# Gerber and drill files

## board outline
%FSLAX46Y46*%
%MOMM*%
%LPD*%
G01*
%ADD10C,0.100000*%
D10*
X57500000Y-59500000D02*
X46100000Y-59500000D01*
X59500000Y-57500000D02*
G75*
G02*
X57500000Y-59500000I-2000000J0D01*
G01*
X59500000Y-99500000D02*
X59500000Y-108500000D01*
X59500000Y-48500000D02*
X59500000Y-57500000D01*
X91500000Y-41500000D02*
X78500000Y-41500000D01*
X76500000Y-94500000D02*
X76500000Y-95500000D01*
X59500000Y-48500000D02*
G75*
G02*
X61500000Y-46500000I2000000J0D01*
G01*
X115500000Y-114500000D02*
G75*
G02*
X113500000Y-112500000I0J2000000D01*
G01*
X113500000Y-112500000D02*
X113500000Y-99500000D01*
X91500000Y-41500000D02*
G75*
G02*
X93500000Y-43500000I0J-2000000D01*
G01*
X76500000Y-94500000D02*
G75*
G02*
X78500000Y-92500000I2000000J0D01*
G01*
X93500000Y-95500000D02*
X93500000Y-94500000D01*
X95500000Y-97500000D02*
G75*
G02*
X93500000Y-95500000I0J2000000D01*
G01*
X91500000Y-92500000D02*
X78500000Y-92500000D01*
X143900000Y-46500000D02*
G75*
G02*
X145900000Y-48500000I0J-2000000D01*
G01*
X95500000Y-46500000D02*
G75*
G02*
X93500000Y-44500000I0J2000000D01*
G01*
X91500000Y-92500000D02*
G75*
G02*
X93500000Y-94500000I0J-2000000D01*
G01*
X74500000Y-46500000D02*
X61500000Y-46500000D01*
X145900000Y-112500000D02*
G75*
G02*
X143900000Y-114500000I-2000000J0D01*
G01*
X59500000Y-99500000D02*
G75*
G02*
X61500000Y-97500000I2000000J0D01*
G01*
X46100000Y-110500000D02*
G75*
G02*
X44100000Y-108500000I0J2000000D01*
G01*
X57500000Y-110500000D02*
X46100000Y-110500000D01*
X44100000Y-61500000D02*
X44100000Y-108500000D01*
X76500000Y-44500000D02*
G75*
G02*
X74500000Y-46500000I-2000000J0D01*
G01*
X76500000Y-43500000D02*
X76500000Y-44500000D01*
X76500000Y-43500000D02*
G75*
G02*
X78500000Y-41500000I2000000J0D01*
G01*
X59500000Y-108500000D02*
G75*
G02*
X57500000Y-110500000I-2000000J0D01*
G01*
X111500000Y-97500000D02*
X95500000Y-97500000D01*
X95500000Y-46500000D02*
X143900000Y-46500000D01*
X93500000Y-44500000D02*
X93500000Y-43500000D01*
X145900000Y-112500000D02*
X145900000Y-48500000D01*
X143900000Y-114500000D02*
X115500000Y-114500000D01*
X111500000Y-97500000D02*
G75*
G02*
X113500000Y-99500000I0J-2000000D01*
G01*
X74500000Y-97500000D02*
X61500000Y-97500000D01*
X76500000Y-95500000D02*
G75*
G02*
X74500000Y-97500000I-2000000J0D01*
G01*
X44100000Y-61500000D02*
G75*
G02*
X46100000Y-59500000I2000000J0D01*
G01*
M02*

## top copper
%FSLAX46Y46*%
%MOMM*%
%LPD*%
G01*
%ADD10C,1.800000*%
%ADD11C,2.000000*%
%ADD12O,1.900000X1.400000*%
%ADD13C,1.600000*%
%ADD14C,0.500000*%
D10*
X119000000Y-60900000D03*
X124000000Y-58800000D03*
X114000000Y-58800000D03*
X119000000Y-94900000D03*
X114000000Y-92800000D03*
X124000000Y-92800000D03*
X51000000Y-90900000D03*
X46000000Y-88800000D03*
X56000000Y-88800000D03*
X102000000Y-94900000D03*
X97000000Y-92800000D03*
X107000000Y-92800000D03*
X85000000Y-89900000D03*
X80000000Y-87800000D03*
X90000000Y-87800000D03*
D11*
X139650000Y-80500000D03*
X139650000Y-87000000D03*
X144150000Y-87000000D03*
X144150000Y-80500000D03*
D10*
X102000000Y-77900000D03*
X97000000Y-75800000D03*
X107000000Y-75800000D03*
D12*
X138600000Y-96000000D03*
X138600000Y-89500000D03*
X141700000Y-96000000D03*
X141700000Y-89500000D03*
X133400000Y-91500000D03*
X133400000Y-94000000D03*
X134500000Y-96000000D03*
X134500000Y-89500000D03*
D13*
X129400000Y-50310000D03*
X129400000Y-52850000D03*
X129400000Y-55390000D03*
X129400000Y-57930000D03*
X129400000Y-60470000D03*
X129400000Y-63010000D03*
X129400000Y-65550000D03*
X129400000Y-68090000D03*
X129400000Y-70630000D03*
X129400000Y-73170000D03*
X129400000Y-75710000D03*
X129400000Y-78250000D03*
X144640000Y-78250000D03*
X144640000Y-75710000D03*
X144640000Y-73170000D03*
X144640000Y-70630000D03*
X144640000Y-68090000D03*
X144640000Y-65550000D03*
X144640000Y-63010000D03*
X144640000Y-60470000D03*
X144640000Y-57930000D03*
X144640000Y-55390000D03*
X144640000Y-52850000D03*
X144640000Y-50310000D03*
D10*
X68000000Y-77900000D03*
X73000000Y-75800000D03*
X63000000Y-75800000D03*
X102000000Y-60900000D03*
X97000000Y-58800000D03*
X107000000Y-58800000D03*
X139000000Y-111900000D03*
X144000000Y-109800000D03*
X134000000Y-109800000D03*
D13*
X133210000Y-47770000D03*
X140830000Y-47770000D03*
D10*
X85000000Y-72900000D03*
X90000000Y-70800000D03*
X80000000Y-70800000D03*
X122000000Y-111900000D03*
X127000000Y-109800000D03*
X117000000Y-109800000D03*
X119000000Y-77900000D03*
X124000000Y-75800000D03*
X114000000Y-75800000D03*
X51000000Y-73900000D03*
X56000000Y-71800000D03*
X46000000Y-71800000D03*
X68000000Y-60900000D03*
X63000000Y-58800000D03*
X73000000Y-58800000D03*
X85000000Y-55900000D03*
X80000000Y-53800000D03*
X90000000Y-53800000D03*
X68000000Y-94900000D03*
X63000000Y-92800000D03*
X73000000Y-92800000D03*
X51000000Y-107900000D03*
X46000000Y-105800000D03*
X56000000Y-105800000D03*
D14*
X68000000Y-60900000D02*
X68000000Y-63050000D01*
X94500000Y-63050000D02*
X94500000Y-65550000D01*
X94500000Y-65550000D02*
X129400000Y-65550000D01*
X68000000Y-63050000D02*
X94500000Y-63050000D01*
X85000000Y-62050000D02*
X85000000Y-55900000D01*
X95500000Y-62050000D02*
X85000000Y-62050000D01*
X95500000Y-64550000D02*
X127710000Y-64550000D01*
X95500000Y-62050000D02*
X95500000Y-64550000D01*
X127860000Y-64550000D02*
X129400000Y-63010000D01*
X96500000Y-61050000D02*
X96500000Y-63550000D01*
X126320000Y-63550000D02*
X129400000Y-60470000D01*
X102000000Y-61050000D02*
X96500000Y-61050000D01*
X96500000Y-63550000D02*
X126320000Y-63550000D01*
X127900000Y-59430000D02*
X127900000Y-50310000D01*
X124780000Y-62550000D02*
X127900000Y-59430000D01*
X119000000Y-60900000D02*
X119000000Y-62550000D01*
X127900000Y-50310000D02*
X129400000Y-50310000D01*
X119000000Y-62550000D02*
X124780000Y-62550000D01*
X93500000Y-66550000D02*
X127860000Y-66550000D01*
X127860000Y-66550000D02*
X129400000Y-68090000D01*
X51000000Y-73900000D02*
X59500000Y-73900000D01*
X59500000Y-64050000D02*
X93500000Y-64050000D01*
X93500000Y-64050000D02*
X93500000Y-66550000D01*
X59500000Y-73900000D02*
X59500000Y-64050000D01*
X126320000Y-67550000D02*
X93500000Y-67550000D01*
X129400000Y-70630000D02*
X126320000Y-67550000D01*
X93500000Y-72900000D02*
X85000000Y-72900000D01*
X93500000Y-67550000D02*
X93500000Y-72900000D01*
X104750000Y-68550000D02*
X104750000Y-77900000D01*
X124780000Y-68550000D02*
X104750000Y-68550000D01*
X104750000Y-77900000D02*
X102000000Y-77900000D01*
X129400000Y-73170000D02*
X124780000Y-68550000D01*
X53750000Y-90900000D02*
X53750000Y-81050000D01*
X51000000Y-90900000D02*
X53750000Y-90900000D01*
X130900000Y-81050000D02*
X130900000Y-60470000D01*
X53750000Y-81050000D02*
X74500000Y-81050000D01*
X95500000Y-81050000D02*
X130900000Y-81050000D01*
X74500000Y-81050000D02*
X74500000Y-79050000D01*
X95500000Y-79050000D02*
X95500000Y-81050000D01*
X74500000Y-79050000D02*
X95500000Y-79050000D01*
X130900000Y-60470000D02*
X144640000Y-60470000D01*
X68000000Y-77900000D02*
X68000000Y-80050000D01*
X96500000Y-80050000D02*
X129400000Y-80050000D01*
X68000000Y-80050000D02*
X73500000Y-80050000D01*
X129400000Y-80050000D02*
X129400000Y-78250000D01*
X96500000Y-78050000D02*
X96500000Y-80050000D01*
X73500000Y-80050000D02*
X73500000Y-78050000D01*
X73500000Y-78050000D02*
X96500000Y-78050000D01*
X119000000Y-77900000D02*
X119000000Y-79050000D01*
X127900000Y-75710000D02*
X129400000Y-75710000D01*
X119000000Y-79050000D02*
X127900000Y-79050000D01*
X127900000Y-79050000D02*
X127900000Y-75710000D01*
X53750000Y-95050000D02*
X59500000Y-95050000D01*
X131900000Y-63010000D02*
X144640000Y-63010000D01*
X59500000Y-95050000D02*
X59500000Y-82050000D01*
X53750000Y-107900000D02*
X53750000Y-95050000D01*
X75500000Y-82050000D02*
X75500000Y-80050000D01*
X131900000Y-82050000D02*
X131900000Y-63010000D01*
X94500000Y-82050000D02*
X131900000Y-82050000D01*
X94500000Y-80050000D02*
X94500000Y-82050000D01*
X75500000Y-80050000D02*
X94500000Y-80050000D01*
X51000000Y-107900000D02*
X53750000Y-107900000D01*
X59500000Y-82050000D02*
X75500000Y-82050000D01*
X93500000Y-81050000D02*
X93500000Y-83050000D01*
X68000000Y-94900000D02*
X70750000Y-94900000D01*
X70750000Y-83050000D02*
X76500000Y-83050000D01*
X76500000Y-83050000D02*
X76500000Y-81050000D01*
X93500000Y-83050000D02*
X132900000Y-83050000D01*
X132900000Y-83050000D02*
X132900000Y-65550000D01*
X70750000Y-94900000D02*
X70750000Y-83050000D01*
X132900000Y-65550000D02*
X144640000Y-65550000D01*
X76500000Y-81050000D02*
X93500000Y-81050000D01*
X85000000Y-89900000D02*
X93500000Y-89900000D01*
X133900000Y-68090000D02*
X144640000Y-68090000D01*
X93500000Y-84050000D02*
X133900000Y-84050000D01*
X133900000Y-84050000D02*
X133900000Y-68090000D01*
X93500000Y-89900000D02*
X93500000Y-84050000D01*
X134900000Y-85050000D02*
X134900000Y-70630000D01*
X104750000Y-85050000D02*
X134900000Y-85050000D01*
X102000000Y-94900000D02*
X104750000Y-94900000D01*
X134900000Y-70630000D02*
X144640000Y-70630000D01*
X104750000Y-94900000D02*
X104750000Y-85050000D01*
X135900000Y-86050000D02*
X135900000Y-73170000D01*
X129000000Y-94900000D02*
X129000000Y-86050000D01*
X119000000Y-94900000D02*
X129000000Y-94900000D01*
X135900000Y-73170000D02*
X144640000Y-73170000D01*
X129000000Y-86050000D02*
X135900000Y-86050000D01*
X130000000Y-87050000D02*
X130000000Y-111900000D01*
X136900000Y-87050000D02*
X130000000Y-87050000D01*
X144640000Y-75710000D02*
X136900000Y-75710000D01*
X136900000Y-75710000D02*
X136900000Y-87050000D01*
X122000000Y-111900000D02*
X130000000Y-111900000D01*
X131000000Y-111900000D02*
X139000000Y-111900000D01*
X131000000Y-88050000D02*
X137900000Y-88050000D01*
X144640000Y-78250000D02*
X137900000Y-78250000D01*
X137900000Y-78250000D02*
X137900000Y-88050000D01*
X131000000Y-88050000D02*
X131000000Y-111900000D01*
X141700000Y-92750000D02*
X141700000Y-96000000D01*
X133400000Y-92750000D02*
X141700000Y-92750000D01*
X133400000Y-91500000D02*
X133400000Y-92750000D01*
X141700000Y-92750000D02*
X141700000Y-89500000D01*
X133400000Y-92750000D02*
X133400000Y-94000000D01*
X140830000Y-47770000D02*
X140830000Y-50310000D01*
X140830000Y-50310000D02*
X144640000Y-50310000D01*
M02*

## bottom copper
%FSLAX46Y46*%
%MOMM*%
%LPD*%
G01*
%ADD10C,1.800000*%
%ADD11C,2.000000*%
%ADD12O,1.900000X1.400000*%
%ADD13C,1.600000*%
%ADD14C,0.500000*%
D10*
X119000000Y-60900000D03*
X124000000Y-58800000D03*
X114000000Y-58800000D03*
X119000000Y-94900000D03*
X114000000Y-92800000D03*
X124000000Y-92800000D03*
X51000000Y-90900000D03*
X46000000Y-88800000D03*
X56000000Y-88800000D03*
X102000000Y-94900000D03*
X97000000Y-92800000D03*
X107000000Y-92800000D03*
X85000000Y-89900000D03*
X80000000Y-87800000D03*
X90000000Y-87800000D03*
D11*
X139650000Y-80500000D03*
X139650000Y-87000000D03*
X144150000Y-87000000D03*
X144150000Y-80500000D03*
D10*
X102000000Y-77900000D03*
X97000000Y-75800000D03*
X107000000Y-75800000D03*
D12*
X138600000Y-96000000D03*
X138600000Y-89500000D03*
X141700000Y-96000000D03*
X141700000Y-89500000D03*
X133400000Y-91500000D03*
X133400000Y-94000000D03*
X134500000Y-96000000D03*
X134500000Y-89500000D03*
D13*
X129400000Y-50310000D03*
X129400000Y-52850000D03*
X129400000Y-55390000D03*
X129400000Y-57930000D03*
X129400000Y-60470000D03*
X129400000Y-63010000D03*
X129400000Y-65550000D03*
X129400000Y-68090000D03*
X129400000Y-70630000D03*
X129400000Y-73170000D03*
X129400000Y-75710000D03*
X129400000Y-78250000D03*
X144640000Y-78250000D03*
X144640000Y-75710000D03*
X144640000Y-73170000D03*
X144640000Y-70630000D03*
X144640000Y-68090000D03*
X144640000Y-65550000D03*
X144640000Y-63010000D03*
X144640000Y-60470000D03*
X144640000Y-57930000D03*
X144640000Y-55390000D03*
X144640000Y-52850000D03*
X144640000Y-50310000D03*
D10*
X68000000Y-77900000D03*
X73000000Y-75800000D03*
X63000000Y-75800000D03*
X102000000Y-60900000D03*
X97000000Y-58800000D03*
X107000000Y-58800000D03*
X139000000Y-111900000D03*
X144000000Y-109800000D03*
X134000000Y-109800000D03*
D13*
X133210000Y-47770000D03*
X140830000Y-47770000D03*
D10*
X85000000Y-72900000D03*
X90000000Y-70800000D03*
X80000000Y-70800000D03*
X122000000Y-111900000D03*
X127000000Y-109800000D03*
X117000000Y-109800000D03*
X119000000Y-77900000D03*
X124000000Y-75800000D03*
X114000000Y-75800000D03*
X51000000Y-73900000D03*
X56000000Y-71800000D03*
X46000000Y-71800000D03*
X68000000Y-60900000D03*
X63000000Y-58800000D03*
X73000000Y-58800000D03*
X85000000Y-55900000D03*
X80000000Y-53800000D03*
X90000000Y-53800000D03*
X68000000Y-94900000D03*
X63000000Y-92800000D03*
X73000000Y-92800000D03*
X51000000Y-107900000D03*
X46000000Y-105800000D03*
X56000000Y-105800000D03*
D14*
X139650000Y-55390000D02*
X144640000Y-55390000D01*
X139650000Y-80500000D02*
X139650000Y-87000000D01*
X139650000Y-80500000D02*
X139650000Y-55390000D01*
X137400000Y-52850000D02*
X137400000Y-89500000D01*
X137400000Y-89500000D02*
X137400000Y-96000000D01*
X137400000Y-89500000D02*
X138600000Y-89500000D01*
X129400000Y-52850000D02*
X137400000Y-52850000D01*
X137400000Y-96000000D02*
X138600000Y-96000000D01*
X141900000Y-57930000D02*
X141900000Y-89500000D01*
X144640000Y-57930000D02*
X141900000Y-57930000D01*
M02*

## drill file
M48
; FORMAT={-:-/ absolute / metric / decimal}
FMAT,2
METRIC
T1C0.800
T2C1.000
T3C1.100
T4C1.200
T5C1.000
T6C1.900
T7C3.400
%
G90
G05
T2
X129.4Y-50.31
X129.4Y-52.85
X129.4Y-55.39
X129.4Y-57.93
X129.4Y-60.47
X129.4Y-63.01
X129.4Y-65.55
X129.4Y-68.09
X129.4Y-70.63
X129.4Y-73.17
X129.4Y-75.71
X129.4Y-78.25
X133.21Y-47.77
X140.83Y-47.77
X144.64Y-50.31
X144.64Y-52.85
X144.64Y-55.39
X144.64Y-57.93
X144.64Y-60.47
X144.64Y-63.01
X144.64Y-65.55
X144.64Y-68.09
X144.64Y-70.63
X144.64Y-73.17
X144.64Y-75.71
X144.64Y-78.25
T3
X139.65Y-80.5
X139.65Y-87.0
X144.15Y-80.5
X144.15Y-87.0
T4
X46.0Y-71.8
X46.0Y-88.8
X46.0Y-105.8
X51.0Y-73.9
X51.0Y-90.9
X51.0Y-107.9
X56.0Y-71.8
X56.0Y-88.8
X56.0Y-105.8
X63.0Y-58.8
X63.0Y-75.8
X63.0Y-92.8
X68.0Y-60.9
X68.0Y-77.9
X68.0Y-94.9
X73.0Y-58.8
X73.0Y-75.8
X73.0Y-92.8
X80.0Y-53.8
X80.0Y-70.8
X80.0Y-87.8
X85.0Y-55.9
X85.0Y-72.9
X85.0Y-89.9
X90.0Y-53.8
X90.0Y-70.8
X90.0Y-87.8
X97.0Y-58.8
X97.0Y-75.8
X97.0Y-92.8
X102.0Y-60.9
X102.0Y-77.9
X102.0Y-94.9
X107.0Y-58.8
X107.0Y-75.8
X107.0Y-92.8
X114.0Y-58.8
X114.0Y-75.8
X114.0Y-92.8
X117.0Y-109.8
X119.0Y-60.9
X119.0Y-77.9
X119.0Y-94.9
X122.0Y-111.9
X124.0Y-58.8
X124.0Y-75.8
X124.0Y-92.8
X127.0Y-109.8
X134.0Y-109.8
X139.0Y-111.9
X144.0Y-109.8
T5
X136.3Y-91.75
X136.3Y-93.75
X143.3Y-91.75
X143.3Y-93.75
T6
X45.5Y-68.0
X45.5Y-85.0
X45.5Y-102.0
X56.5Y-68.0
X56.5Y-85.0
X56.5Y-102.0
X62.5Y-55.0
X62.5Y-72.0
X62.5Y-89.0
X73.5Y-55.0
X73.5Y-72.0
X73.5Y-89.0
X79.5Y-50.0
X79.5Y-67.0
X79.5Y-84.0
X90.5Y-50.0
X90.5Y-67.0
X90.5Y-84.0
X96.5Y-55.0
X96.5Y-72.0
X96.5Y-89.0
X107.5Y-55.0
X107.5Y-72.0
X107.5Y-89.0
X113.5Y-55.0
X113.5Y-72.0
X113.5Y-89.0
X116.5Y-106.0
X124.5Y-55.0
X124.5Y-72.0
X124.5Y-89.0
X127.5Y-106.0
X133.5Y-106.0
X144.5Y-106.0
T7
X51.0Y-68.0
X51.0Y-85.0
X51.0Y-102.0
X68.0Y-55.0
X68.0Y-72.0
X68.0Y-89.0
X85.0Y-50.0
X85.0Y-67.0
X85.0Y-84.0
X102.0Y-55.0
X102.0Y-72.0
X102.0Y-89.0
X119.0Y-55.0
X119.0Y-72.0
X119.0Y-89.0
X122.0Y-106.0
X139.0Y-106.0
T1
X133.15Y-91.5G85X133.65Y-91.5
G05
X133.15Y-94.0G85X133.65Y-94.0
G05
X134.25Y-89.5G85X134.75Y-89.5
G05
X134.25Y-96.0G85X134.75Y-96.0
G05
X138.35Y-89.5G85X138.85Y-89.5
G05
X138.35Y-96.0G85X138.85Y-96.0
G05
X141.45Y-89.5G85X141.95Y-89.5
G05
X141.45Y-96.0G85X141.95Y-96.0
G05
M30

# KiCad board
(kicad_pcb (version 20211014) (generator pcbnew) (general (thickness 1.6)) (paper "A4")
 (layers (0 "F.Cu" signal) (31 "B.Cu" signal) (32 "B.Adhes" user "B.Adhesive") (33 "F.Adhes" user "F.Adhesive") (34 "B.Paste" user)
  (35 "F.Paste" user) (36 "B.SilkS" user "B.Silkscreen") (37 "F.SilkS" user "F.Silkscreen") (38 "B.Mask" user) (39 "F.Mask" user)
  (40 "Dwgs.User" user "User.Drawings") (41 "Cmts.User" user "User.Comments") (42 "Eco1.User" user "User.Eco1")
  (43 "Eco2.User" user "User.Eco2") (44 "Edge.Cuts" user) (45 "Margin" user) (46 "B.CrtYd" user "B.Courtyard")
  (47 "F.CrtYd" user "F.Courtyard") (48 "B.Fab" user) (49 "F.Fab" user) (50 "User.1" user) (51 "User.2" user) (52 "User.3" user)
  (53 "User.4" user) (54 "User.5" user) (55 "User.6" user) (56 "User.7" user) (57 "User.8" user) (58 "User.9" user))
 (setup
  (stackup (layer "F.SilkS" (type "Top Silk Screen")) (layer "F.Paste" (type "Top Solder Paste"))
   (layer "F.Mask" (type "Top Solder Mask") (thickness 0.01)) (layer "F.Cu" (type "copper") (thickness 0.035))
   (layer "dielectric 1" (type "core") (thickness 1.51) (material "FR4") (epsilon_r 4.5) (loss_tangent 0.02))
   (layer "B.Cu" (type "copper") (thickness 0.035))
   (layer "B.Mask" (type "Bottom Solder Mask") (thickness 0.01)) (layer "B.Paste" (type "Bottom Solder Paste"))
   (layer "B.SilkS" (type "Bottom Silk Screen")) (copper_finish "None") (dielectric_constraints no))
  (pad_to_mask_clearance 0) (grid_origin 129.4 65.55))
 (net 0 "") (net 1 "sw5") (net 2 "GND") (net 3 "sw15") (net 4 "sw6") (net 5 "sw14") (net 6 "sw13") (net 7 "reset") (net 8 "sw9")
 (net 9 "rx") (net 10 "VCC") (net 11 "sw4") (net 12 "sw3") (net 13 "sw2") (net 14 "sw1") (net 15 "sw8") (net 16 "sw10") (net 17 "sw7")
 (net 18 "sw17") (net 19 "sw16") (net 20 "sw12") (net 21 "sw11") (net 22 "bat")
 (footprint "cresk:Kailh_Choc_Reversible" (layer "F.Cu") (at 119 55)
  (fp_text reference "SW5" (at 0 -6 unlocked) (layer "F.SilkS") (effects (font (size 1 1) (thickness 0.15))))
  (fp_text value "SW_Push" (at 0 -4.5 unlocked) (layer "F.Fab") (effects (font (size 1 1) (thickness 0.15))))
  (pad "" np_thru_hole circle (at 0 0) (size 3.4 3.4) (drill 3.4) (layers *.Mask))
  (pad "" np_thru_hole circle (at -5.5 0) (size 1.9 1.9) (drill 1.9) (layers *.Mask))
  (pad "" np_thru_hole circle (at 5.5 0) (size 1.9 1.9) (drill 1.9) (layers *.Mask))
  (pad "1" thru_hole circle (at 0 5.9) (size 1.8 1.8) (drill 1.2) (layers *.Cu *.Mask) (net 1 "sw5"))
  (pad "2" thru_hole circle (at 5 3.8) (size 1.8 1.8) (drill 1.2) (layers *.Cu *.Mask) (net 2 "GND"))
  (pad "2" thru_hole circle (at -5 3.8) (size 1.8 1.8) (drill 1.2) (layers *.Cu *.Mask) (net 2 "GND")))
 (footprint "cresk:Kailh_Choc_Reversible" (layer "F.Cu") (at 119 89)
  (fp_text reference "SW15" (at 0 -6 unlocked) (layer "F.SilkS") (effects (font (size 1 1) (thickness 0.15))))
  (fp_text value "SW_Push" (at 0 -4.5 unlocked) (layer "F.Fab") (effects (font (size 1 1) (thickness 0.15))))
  (pad "" np_thru_hole circle (at 5.5 0) (size 1.9 1.9) (drill 1.9) (layers *.Mask))
  (pad "" np_thru_hole circle (at 0 0) (size 3.4 3.4) (drill 3.4) (layers *.Mask))
  (pad "" np_thru_hole circle (at -5.5 0) (size 1.9 1.9) (drill 1.9) (layers *.Mask))
  (pad "1" thru_hole circle (at 0 5.9) (size 1.8 1.8) (drill 1.2) (layers *.Cu *.Mask) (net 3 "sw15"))
  (pad "2" thru_hole circle (at -5 3.8) (size 1.8 1.8) (drill 1.2) (layers *.Cu *.Mask) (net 2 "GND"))
  (pad "2" thru_hole circle (at 5 3.8) (size 1.8 1.8) (drill 1.2) (layers *.Cu *.Mask) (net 2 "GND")))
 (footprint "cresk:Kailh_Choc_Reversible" (layer "F.Cu") (at 51 85)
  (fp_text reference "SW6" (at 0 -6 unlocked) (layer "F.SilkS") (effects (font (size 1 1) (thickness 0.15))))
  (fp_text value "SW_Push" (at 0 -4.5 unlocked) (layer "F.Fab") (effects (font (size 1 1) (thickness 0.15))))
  (pad "" np_thru_hole circle (at 0 0) (size 3.4 3.4) (drill 3.4) (layers *.Mask))
  (pad "" np_thru_hole circle (at 5.5 0) (size 1.9 1.9) (drill 1.9) (layers *.Mask))
  (pad "" np_thru_hole circle (at -5.5 0) (size 1.9 1.9) (drill 1.9) (layers *.Mask))
  (pad "1" thru_hole circle (at 0 5.9) (size 1.8 1.8) (drill 1.2) (layers *.Cu *.Mask) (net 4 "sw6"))
  (pad "2" thru_hole circle (at -5 3.8) (size 1.8 1.8) (drill 1.2) (layers *.Cu *.Mask) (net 2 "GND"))
  (pad "2" thru_hole circle (at 5 3.8) (size 1.8 1.8) (drill 1.2) (layers *.Cu *.Mask) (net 2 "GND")))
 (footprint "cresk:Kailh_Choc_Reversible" (layer "F.Cu") (at 102 89)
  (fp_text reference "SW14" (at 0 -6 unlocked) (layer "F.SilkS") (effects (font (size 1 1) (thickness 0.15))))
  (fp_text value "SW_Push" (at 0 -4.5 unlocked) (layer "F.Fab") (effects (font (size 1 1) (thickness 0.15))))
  (pad "" np_thru_hole circle (at -5.5 0) (size 1.9 1.9) (drill 1.9) (layers *.Mask))
  (pad "" np_thru_hole circle (at 0 0) (size 3.4 3.4) (drill 3.4) (layers *.Mask))
  (pad "" np_thru_hole circle (at 5.5 0) (size 1.9 1.9) (drill 1.9) (layers *.Mask))
  (pad "1" thru_hole circle (at 0 5.9) (size 1.8 1.8) (drill 1.2) (layers *.Cu *.Mask) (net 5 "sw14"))
  (pad "2" thru_hole circle (at -5 3.8) (size 1.8 1.8) (drill 1.2) (layers *.Cu *.Mask) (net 2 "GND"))
  (pad "2" thru_hole circle (at 5 3.8) (size 1.8 1.8) (drill 1.2) (layers *.Cu *.Mask) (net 2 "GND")))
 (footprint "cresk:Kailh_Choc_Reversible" (layer "F.Cu") (at 85 84)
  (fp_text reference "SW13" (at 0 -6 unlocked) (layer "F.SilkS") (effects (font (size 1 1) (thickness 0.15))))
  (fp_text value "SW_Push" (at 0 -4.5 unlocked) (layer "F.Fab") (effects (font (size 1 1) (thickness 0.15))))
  (pad "" np_thru_hole circle (at 0 0) (size 3.4 3.4) (drill 3.4) (layers *.Mask))
  (pad "" np_thru_hole circle (at -5.5 0) (size 1.9 1.9) (drill 1.9) (layers *.Mask))
  (pad "" np_thru_hole circle (at 5.5 0) (size 1.9 1.9) (drill 1.9) (layers *.Mask))
  (pad "1" thru_hole circle (at 0 5.9) (size 1.8 1.8) (drill 1.2) (layers *.Cu *.Mask) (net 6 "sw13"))
  (pad "2" thru_hole circle (at -5 3.8) (size 1.8 1.8) (drill 1.2) (layers *.Cu *.Mask) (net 2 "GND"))
  (pad "2" thru_hole circle (at 5 3.8) (size 1.8 1.8) (drill 1.2) (layers *.Cu *.Mask) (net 2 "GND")))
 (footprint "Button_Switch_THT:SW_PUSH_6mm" (layer "F.Cu") (at 139.65 87 90)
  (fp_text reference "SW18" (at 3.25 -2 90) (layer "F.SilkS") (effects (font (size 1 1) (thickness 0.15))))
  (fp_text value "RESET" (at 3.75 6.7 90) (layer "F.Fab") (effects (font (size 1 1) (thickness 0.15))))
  (pad "1" thru_hole circle (at 6.5 0 180) (size 2 2) (drill 1.1) (layers *.Cu *.Mask) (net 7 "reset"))
  (pad "1" thru_hole circle (at 0 0 180) (size 2 2) (drill 1.1) (layers *.Cu *.Mask) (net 7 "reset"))
  (pad "2" thru_hole circle (at 0 4.5 180) (size 2 2) (drill 1.1) (layers *.Cu *.Mask) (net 2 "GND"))
  (pad "2" thru_hole circle (at 6.5 4.5 180) (size 2 2) (drill 1.1) (layers *.Cu *.Mask) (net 2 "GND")))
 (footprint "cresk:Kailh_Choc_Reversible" (layer "F.Cu") (at 102 72)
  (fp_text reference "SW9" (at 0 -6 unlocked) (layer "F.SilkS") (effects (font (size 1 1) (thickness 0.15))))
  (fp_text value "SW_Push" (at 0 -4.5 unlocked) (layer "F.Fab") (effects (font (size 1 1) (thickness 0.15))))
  (pad "" np_thru_hole circle (at -5.5 0) (size 1.9 1.9) (drill 1.9) (layers *.Mask))
  (pad "" np_thru_hole circle (at 0 0) (size 3.4 3.4) (drill 3.4) (layers *.Mask))
  (pad "" np_thru_hole circle (at 5.5 0) (size 1.9 1.9) (drill 1.9) (layers *.Mask))
  (pad "1" thru_hole circle (at 0 5.9) (size 1.8 1.8) (drill 1.2) (layers *.Cu *.Mask) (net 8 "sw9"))
  (pad "2" thru_hole circle (at -5 3.8) (size 1.8 1.8) (drill 1.2) (layers *.Cu *.Mask) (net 2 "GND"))
  (pad "2" thru_hole circle (at 5 3.8) (size 1.8 1.8) (drill 1.2) (layers *.Cu *.Mask) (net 2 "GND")))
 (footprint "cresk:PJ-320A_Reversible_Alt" (layer "F.Cu") (at 133.4 96 90)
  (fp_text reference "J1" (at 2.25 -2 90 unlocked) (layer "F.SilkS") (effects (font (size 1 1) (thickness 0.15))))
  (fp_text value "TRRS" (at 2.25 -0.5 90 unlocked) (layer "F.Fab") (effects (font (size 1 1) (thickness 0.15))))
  (pad "" np_thru_hole circle (at 2.25 2.9 90) (size 1 1) (drill 1) (layers *.Mask))
  (pad "" np_thru_hole circle (at 4.25 2.9 90) (size 1 1) (drill 1) (layers *.Mask))
  (pad "" np_thru_hole circle (at 2.25 9.9 90) (size 1 1) (drill 1) (layers *.Mask))
  (pad "" np_thru_hole circle (at 4.25 9.9 90) (size 1 1) (drill 1) (layers *.Mask))
  (pad "R1" thru_hole oval (at 0 5.2 90) (size 1.4 1.9) (drill oval 0.8 1.3) (layers *.Cu *.Mask) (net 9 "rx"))
  (pad "R1" thru_hole oval (at 6.5 5.2 90) (size 1.4 1.9) (drill oval 0.8 1.3) (layers *.Cu *.Mask) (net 9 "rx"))
  (pad "R2" thru_hole oval (at 0 8.3 90) (size 1.4 1.9) (drill oval 0.8 1.3) (layers *.Cu *.Mask) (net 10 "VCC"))
  (pad "R2" thru_hole oval (at 6.5 8.3 90) (size 1.4 1.9) (drill oval 0.8 1.3) (layers *.Cu *.Mask) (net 10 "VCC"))
  (pad "S" thru_hole oval (at 4.5 0 90) (size 1.4 1.9) (drill oval 0.8 1.3) (layers *.Cu *.Mask) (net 10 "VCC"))
  (pad "S" thru_hole oval (at 2 0 90) (size 1.4 1.9) (drill oval 0.8 1.3) (layers *.Cu *.Mask) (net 10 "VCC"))
  (pad "T" thru_hole oval (at 0 1.1 90) (size 1.4 1.9) (drill oval 0.8 1.3) (layers *.Cu *.Mask) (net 2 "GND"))
  (pad "T" thru_hole oval (at 6.5 1.1 90) (size 1.4 1.9) (drill oval 0.8 1.3) (layers *.Cu *.Mask) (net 2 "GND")))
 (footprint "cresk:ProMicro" (layer "F.Cu") (at 129.4 50.31)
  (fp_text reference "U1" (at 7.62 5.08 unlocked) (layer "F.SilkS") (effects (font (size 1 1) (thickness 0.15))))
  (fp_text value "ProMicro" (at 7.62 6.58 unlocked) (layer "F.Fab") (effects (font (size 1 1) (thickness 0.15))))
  (pad "1" thru_hole circle (at 0 0) (size 1.6 1.6) (drill 1) (layers *.Cu *.Mask) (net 1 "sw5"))
  (pad "2" thru_hole circle (at 0 2.54) (size 1.6 1.6) (drill 1) (layers *.Cu *.Mask) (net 9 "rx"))
  (pad "3" thru_hole circle (at 0 5.08) (size 1.6 1.6) (drill 1) (layers *.Cu *.Mask) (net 2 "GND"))
  (pad "4" thru_hole circle (at 0 7.62) (size 1.6 1.6) (drill 1) (layers *.Cu *.Mask) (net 2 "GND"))
  (pad "5" thru_hole circle (at 0 10.16) (size 1.6 1.6) (drill 1) (layers *.Cu *.Mask) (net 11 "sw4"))
  (pad "6" thru_hole circle (at 0 12.7) (size 1.6 1.6) (drill 1) (layers *.Cu *.Mask) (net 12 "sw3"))
  (pad "7" thru_hole circle (at 0 15.24) (size 1.6 1.6) (drill 1) (layers *.Cu *.Mask) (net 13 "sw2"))
  (pad "8" thru_hole circle (at 0 17.78) (size 1.6 1.6) (drill 1) (layers *.Cu *.Mask) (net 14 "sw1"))
  (pad "9" thru_hole circle (at 0 20.32) (size 1.6 1.6) (drill 1) (layers *.Cu *.Mask) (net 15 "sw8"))
  (pad "10" thru_hole circle (at 0 22.86) (size 1.6 1.6) (drill 1) (layers *.Cu *.Mask) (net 8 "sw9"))
  (pad "11" thru_hole circle (at 0 25.4) (size 1.6 1.6) (drill 1) (layers *.Cu *.Mask) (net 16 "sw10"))
  (pad "12" thru_hole circle (at 0 27.94) (size 1.6 1.6) (drill 1) (layers *.Cu *.Mask) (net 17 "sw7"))
  (pad "13" thru_hole circle (at 15.24 27.94) (size 1.6 1.6) (drill 1) (layers *.Cu *.Mask) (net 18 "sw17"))
  (pad "14" thru_hole circle (at 15.24 25.4) (size 1.6 1.6) (drill 1) (layers *.Cu *.Mask) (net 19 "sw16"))
  (pad "15" thru_hole circle (at 15.24 22.86) (size 1.6 1.6) (drill 1) (layers *.Cu *.Mask) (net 3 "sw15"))
  (pad "16" thru_hole circle (at 15.24 20.32) (size 1.6 1.6) (drill 1) (layers *.Cu *.Mask) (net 5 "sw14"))
  (pad "17" thru_hole circle (at 15.24 17.78) (size 1.6 1.6) (drill 1) (layers *.Cu *.Mask) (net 6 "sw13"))
  (pad "18" thru_hole circle (at 15.24 15.24) (size 1.6 1.6) (drill 1) (layers *.Cu *.Mask) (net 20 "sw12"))
  (pad "19" thru_hole circle (at 15.24 12.7) (size 1.6 1.6) (drill 1) (layers *.Cu *.Mask) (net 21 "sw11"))
  (pad "20" thru_hole circle (at 15.24 10.16) (size 1.6 1.6) (drill 1) (layers *.Cu *.Mask) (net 4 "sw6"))
  (pad "21" thru_hole circle (at 15.24 7.62) (size 1.6 1.6) (drill 1) (layers *.Cu *.Mask) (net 10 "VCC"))
  (pad "22" thru_hole circle (at 15.24 5.08) (size 1.6 1.6) (drill 1) (layers *.Cu *.Mask) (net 7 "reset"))
  (pad "23" thru_hole circle (at 15.24 2.54) (size 1.6 1.6) (drill 1) (layers *.Cu *.Mask) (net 2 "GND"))
  (pad "24" thru_hole circle (at 15.24 0) (size 1.6 1.6) (drill 1) (layers *.Cu *.Mask) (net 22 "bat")))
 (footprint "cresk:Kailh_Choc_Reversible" (layer "F.Cu") (at 68 72)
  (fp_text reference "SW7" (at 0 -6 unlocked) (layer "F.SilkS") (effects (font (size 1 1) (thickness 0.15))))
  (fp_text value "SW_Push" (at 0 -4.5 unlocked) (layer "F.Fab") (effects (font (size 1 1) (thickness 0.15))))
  (pad "" np_thru_hole circle (at 5.5 0) (size 1.9 1.9) (drill 1.9) (layers *.Mask))
  (pad "" np_thru_hole circle (at -5.5 0) (size 1.9 1.9) (drill 1.9) (layers *.Mask))
  (pad "" np_thru_hole circle (at 0 0) (size 3.4 3.4) (drill 3.4) (layers *.Mask))
  (pad "1" thru_hole circle (at 0 5.9) (size 1.8 1.8) (drill 1.2) (layers *.Cu *.Mask) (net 17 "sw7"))
  (pad "2" thru_hole circle (at 5 3.8) (size 1.8 1.8) (drill 1.2) (layers *.Cu *.Mask) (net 2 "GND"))
  (pad "2" thru_hole circle (at -5 3.8) (size 1.8 1.8) (drill 1.2) (layers *.Cu *.Mask) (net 2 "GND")))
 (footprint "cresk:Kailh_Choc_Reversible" (layer "F.Cu") (at 102 55)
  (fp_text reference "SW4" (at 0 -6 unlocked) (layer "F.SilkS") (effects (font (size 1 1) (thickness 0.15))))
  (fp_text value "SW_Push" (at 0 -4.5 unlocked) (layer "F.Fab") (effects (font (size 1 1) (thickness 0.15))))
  (pad "" np_thru_hole circle (at 5.5 0) (size 1.9 1.9) (drill 1.9) (layers *.Mask))
  (pad "" np_thru_hole circle (at -5.5 0) (size 1.9 1.9) (drill 1.9) (layers *.Mask))
  (pad "" np_thru_hole circle (at 0 0) (size 3.4 3.4) (drill 3.4) (layers *.Mask))
  (pad "1" thru_hole circle (at 0 5.9) (size 1.8 1.8) (drill 1.2) (layers *.Cu *.Mask) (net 11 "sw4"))
  (pad "2" thru_hole circle (at -5 3.8) (size 1.8 1.8) (drill 1.2) (layers *.Cu *.Mask) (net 2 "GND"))
  (pad "2" thru_hole circle (at 5 3.8) (size 1.8 1.8) (drill 1.2) (layers *.Cu *.Mask) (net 2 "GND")))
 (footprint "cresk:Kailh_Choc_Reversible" (layer "F.Cu") (at 139 106)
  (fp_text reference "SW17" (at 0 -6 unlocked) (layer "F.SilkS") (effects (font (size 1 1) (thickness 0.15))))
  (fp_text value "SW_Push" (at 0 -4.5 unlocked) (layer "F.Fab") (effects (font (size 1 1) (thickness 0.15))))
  (pad "" np_thru_hole circle (at -5.5 0) (size 1.9 1.9) (drill 1.9) (layers *.Mask))
  (pad "" np_thru_hole circle (at 5.5 0) (size 1.9 1.9) (drill 1.9) (layers *.Mask))
  (pad "" np_thru_hole circle (at 0 0) (size 3.4 3.4) (drill 3.4) (layers *.Mask))
  (pad "1" thru_hole circle (at 0 5.9) (size 1.8 1.8) (drill 1.2) (layers *.Cu *.Mask) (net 18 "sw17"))
  (pad "2" thru_hole circle (at 5 3.8) (size 1.8 1.8) (drill 1.2) (layers *.Cu *.Mask) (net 2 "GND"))
  (pad "2" thru_hole circle (at -5 3.8) (size 1.8 1.8) (drill 1.2) (layers *.Cu *.Mask) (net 2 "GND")))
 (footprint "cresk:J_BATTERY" (layer "F.Cu") (at 133.21 47.77)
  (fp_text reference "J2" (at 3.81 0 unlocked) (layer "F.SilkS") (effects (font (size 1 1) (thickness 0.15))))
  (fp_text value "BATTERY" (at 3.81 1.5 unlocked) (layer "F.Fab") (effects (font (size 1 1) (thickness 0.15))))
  (pad "1" thru_hole circle (at 0 0) (size 1.6 1.6) (drill 1) (layers *.Cu *.Mask) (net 2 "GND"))
  (pad "2" thru_hole circle (at 7.62 0) (size 1.6 1.6) (drill 1) (layers *.Cu *.Mask) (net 22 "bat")))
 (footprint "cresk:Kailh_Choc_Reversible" (layer "F.Cu") (at 85 67)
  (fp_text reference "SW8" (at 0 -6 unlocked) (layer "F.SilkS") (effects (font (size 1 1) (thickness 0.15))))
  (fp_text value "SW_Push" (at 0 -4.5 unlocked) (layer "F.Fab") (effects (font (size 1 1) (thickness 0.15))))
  (pad "" np_thru_hole circle (at 0 0) (size 3.4 3.4) (drill 3.4) (layers *.Mask))
  (pad "" np_thru_hole circle (at -5.5 0) (size 1.9 1.9) (drill 1.9) (layers *.Mask))
  (pad "" np_thru_hole circle (at 5.5 0) (size 1.9 1.9) (drill 1.9) (layers *.Mask))
  (pad "1" thru_hole circle (at 0 5.9) (size 1.8 1.8) (drill 1.2) (layers *.Cu *.Mask) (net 15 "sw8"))
  (pad "2" thru_hole circle (at 5 3.8) (size 1.8 1.8) (drill 1.2) (layers *.Cu *.Mask) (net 2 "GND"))
  (pad "2" thru_hole circle (at -5 3.8) (size 1.8 1.8) (drill 1.2) (layers *.Cu *.Mask) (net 2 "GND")))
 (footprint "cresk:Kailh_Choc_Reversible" (layer "F.Cu") (at 122 106)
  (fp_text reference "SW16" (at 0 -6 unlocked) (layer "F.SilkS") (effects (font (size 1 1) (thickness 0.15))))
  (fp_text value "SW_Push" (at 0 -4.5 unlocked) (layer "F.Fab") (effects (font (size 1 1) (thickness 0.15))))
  (pad "" np_thru_hole circle (at 0 0) (size 3.4 3.4) (drill 3.4) (layers *.Mask))
  (pad "" np_thru_hole circle (at -5.5 0) (size 1.9 1.9) (drill 1.9) (layers *.Mask))
  (pad "" np_thru_hole circle (at 5.5 0) (size 1.9 1.9) (drill 1.9) (layers *.Mask))
  (pad "1" thru_hole circle (at 0 5.9) (size 1.8 1.8) (drill 1.2) (layers *.Cu *.Mask) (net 19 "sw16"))
  (pad "2" thru_hole circle (at 5 3.8) (size 1.8 1.8) (drill 1.2) (layers *.Cu *.Mask) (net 2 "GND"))
  (pad "2" thru_hole circle (at -5 3.8) (size 1.8 1.8) (drill 1.2) (layers *.Cu *.Mask) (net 2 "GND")))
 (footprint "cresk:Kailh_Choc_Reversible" (layer "F.Cu") (at 119 72)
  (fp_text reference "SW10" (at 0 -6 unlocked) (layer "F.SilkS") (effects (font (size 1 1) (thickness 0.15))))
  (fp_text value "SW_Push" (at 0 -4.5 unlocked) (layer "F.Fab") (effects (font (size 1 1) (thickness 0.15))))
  (pad "" np_thru_hole circle (at 0 0) (size 3.4 3.4) (drill 3.4) (layers *.Mask))
  (pad "" np_thru_hole circle (at -5.5 0) (size 1.9 1.9) (drill 1.9) (layers *.Mask))
  (pad "" np_thru_hole circle (at 5.5 0) (size 1.9 1.9) (drill 1.9) (layers *.Mask))
  (pad "1" thru_hole circle (at 0 5.9) (size 1.8 1.8) (drill 1.2) (layers *.Cu *.Mask) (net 16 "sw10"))
  (pad "2" thru_hole circle (at 5 3.8) (size 1.8 1.8) (drill 1.2) (layers *.Cu *.Mask) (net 2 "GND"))
  (pad "2" thru_hole circle (at -5 3.8) (size 1.8 1.8) (drill 1.2) (layers *.Cu *.Mask) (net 2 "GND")))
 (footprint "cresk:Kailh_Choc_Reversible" (layer "F.Cu") (at 51 68)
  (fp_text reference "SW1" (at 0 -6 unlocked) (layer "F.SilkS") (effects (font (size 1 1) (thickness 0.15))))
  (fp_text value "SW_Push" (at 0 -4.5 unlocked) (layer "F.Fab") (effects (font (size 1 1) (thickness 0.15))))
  (pad "" np_thru_hole circle (at -5.5 0) (size 1.9 1.9) (drill 1.9) (layers *.Mask))
  (pad "" np_thru_hole circle (at 5.5 0) (size 1.9 1.9) (drill 1.9) (layers *.Mask))
  (pad "" np_thru_hole circle (at 0 0) (size 3.4 3.4) (drill 3.4) (layers *.Mask))
  (pad "1" thru_hole circle (at 0 5.9) (size 1.8 1.8) (drill 1.2) (layers *.Cu *.Mask) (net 14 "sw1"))
  (pad "2" thru_hole circle (at 5 3.8) (size 1.8 1.8) (drill 1.2) (layers *.Cu *.Mask) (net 2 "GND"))
  (pad "2" thru_hole circle (at -5 3.8) (size 1.8 1.8) (drill 1.2) (layers *.Cu *.Mask) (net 2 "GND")))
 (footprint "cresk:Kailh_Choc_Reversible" (layer "F.Cu") (at 68 55)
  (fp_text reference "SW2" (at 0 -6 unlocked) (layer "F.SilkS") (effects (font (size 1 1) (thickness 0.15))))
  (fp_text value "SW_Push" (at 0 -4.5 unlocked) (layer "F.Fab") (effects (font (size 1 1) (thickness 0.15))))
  (pad "" np_thru_hole circle (at 0 0) (size 3.4 3.4) (drill 3.4) (layers *.Mask))
  (pad "" np_thru_hole circle (at -5.5 0) (size 1.9 1.9) (drill 1.9) (layers *.Mask))
  (pad "" np_thru_hole circle (at 5.5 0) (size 1.9 1.9) (drill 1.9) (layers *.Mask))
  (pad "1" thru_hole circle (at 0 5.9) (size 1.8 1.8) (drill 1.2) (layers *.Cu *.Mask) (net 13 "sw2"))
  (pad "2" thru_hole circle (at -5 3.8) (size 1.8 1.8) (drill 1.2) (layers *.Cu *.Mask) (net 2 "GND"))
  (pad "2" thru_hole circle (at 5 3.8) (size 1.8 1.8) (drill 1.2) (layers *.Cu *.Mask) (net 2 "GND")))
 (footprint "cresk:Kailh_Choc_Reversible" (layer "F.Cu") (at 85 50)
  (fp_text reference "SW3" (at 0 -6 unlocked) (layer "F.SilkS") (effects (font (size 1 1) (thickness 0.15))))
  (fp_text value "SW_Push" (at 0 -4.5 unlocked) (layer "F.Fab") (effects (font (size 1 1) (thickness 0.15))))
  (pad "" np_thru_hole circle (at 0 0) (size 3.4 3.4) (drill 3.4) (layers *.Mask))
  (pad "" np_thru_hole circle (at -5.5 0) (size 1.9 1.9) (drill 1.9) (layers *.Mask))
  (pad "" np_thru_hole circle (at 5.5 0) (size 1.9 1.9) (drill 1.9) (layers *.Mask))
  (pad "1" thru_hole circle (at 0 5.9) (size 1.8 1.8) (drill 1.2) (layers *.Cu *.Mask) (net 12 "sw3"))
  (pad "2" thru_hole circle (at -5 3.8) (size 1.8 1.8) (drill 1.2) (layers *.Cu *.Mask) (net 2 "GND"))
  (pad "2" thru_hole circle (at 5 3.8) (size 1.8 1.8) (drill 1.2) (layers *.Cu *.Mask) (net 2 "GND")))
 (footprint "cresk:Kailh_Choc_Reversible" (layer "F.Cu") (at 68 89)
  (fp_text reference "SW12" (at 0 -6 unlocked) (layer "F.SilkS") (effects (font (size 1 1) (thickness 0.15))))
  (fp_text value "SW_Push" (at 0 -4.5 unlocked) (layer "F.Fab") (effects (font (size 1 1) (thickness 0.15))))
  (pad "" np_thru_hole circle (at 0 0) (size 3.4 3.4) (drill 3.4) (layers *.Mask))
  (pad "" np_thru_hole circle (at -5.5 0) (size 1.9 1.9) (drill 1.9) (layers *.Mask))
  (pad "" np_thru_hole circle (at 5.5 0) (size 1.9 1.9) (drill 1.9) (layers *.Mask))
  (pad "1" thru_hole circle (at 0 5.9) (size 1.8 1.8) (drill 1.2) (layers *.Cu *.Mask) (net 20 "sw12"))
  (pad "2" thru_hole circle (at -5 3.8) (size 1.8 1.8) (drill 1.2) (layers *.Cu *.Mask) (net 2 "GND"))
  (pad "2" thru_hole circle (at 5 3.8) (size 1.8 1.8) (drill 1.2) (layers *.Cu *.Mask) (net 2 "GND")))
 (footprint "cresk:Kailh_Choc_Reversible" (layer "F.Cu") (at 51 102)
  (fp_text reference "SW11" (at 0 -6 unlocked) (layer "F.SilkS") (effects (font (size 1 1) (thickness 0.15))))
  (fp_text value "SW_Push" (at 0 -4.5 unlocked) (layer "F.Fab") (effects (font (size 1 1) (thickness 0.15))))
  (pad "" np_thru_hole circle (at -5.5 0) (size 1.9 1.9) (drill 1.9) (layers *.Mask))
  (pad "" np_thru_hole circle (at 0 0) (size 3.4 3.4) (drill 3.4) (layers *.Mask))
  (pad "" np_thru_hole circle (at 5.5 0) (size 1.9 1.9) (drill 1.9) (layers *.Mask))
  (pad "1" thru_hole circle (at 0 5.9) (size 1.8 1.8) (drill 1.2) (layers *.Cu *.Mask) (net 21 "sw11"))
  (pad "2" thru_hole circle (at -5 3.8) (size 1.8 1.8) (drill 1.2) (layers *.Cu *.Mask) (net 2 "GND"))
  (pad "2" thru_hole circle (at 5 3.8) (size 1.8 1.8) (drill 1.2) (layers *.Cu *.Mask) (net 2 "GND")))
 (gr_line (start 57.5 59.5) (end 46.1 59.5) (layer "Edge.Cuts") (width 0.1))
 (gr_arc (start 59.5 57.5) (mid 58.914214 58.914214) (end 57.5 59.5) (layer "Edge.Cuts") (width 0.1))
 (gr_line (start 59.5 99.5) (end 59.5 108.5) (layer "Edge.Cuts") (width 0.1))
 (gr_line (start 59.5 48.5) (end 59.5 57.5) (layer "Edge.Cuts") (width 0.1))
 (gr_line (start 91.5 41.5) (end 78.5 41.5) (layer "Edge.Cuts") (width 0.1))
 (gr_line (start 76.5 94.5) (end 76.5 95.5) (layer "Edge.Cuts") (width 0.1))
 (gr_arc (start 59.5 48.5) (mid 60.085786 47.085786) (end 61.5 46.5) (layer "Edge.Cuts") (width 0.1))
 (gr_arc (start 115.5 114.5) (mid 114.085786 113.914214) (end 113.5 112.5) (layer "Edge.Cuts") (width 0.1))
 (gr_line (start 113.5 112.5) (end 113.5 99.5) (layer "Edge.Cuts") (width 0.1))
 (gr_arc (start 91.5 41.5) (mid 92.914214 42.085786) (end 93.5 43.5) (layer "Edge.Cuts") (width 0.1))
 (gr_arc (start 76.5 94.5) (mid 77.085786 93.085786) (end 78.5 92.5) (layer "Edge.Cuts") (width 0.1))
 (gr_line (start 93.5 95.5) (end 93.5 94.5) (layer "Edge.Cuts") (width 0.1))
 (gr_arc (start 95.5 97.5) (mid 94.085786 96.914214) (end 93.5 95.5) (layer "Edge.Cuts") (width 0.1))
 (gr_line (start 91.5 92.5) (end 78.5 92.5) (layer "Edge.Cuts") (width 0.1))
 (gr_arc (start 143.9 46.5) (mid 145.314214 47.085786) (end 145.9 48.5) (layer "Edge.Cuts") (width 0.1))
 (gr_arc (start 95.5 46.5) (mid 94.085786 45.914214) (end 93.5 44.5) (layer "Edge.Cuts") (width 0.1))
 (gr_arc (start 91.5 92.5) (mid 92.914214 93.085786) (end 93.5 94.5) (layer "Edge.Cuts") (width 0.1))
 (gr_line (start 74.5 46.5) (end 61.5 46.5) (layer "Edge.Cuts") (width 0.1))
 (gr_arc (start 145.9 112.5) (mid 145.314214 113.914214) (end 143.9 114.5) (layer "Edge.Cuts") (width 0.1))
 (gr_arc (start 59.5 99.5) (mid 60.085786 98.085786) (end 61.5 97.5) (layer "Edge.Cuts") (width 0.1))
 (gr_arc (start 46.1 110.5) (mid 44.685786 109.914214) (end 44.1 108.5) (layer "Edge.Cuts") (width 0.1))
 (gr_line (start 57.5 110.5) (end 46.1 110.5) (layer "Edge.Cuts") (width 0.1))
 (gr_line (start 44.1 61.5) (end 44.1 108.5) (layer "Edge.Cuts") (width 0.1))
 (gr_arc (start 76.5 44.5) (mid 75.914214 45.914214) (end 74.5 46.5) (layer "Edge.Cuts") (width 0.1))
 (gr_line (start 76.5 43.5) (end 76.5 44.5) (layer "Edge.Cuts") (width 0.1))
 (gr_arc (start 76.5 43.5) (mid 77.085786 42.085786) (end 78.5 41.5) (layer "Edge.Cuts") (width 0.1))
 (gr_arc (start 59.5 108.5) (mid 58.914214 109.914214) (end 57.5 110.5) (layer "Edge.Cuts") (width 0.1))
 (gr_line (start 111.5 97.5) (end 95.5 97.5) (layer "Edge.Cuts") (width 0.1))
 (gr_line (start 95.5 46.5) (end 143.9 46.5) (layer "Edge.Cuts") (width 0.1))
 (gr_line (start 93.5 44.5) (end 93.5 43.5) (layer "Edge.Cuts") (width 0.1))
 (gr_line (start 145.9 112.5) (end 145.9 48.5) (layer "Edge.Cuts") (width 0.1))
 (gr_line (start 143.9 114.5) (end 115.5 114.5) (layer "Edge.Cuts") (width 0.1))
 (gr_arc (start 111.5 97.5) (mid 112.914214 98.085786) (end 113.5 99.5) (layer "Edge.Cuts") (width 0.1))
 (gr_line (start 74.5 97.5) (end 61.5 97.5) (layer "Edge.Cuts") (width 0.1))
 (gr_arc (start 76.5 95.5) (mid 75.914214 96.914214) (end 74.5 97.5) (layer "Edge.Cuts") (width 0.1))
 (gr_arc (start 44.1 61.5) (mid 44.685786 60.085786) (end 46.1 59.5) (layer "Edge.Cuts") (width 0.1))
 (segment (start 68 60.9) (end 68 63.05) (width 0.5) (layer "F.Cu") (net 13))
 (segment (start 94.5 63.05) (end 94.5 65.55) (width 0.5) (layer "F.Cu") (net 13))
 (segment (start 94.5 65.55) (end 129.4 65.55) (width 0.5) (layer "F.Cu") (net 13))
 (segment (start 68 63.05) (end 94.5 63.05) (width 0.5) (layer "F.Cu") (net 13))
 (segment (start 85 62.05) (end 85 55.9) (width 0.5) (layer "F.Cu") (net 12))
 (segment (start 95.5 62.05) (end 85 62.05) (width 0.5) (layer "F.Cu") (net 12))
 (segment (start 95.5 64.55) (end 127.71 64.55) (width 0.5) (layer "F.Cu") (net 12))
 (segment (start 95.5 62.05) (end 95.5 64.55) (width 0.5) (layer "F.Cu") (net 12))
 (segment (start 127.86 64.55) (end 129.4 63.01) (width 0.5) (layer "F.Cu") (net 12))
 (segment (start 96.5 61.05) (end 96.5 63.55) (width 0.5) (layer "F.Cu") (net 11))
 (segment (start 126.32 63.55) (end 129.4 60.47) (width 0.5) (layer "F.Cu") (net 11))
 (segment (start 102 61.05) (end 96.5 61.05) (width 0.5) (layer "F.Cu") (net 11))
 (segment (start 96.5 63.55) (end 126.32 63.55) (width 0.5) (layer "F.Cu") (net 11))
 (segment (start 127.9 59.43) (end 127.9 50.31) (width 0.5) (layer "F.Cu") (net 1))
 (segment (start 124.78 62.55) (end 127.9 59.43) (width 0.5) (layer "F.Cu") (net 1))
 (segment (start 119 60.9) (end 119 62.55) (width 0.5) (layer "F.Cu") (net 1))
 (segment (start 127.9 50.31) (end 129.4 50.31) (width 0.5) (layer "F.Cu") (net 1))
 (segment (start 119 62.55) (end 124.78 62.55) (width 0.5) (layer "F.Cu") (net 1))
 (segment (start 93.5 66.55) (end 127.86 66.55) (width 0.5) (layer "F.Cu") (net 14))
 (segment (start 127.86 66.55) (end 129.4 68.09) (width 0.5) (layer "F.Cu") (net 14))
 (segment (start 51 73.9) (end 59.5 73.9) (width 0.5) (layer "F.Cu") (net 14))
 (segment (start 59.5 64.05) (end 93.5 64.05) (width 0.5) (layer "F.Cu") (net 14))
 (segment (start 93.5 64.05) (end 93.5 66.55) (width 0.5) (layer "F.Cu") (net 14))
 (segment (start 59.5 73.9) (end 59.5 64.05) (width 0.5) (layer "F.Cu") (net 14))
 (segment (start 126.32 67.55) (end 93.5 67.55) (width 0.5) (layer "F.Cu") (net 15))
 (segment (start 129.4 70.63) (end 126.32 67.55) (width 0.5) (layer "F.Cu") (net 15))
 (segment (start 93.5 72.9) (end 85 72.9) (width 0.5) (layer "F.Cu") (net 15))
 (segment (start 93.5 67.55) (end 93.5 72.9) (width 0.5) (layer "F.Cu") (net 15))
 (segment (start 104.75 68.55) (end 104.75 77.9) (width 0.5) (layer "F.Cu") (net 8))
 (segment (start 124.78 68.55) (end 104.75 68.55) (width 0.5) (layer "F.Cu") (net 8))
 (segment (start 104.75 77.9) (end 102 77.9) (width 0.5) (layer "F.Cu") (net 8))
 (segment (start 129.4 73.17) (end 124.78 68.55) (width 0.5) (layer "F.Cu") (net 8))
 (segment (start 53.75 90.9) (end 53.75 81.05) (width 0.5) (layer "F.Cu") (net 4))
 (segment (start 51 90.9) (end 53.75 90.9) (width 0.5) (layer "F.Cu") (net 4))
 (segment (start 130.9 81.05) (end 130.9 60.47) (width 0.5) (layer "F.Cu") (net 4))
 (segment (start 53.75 81.05) (end 74.5 81.05) (width 0.5) (layer "F.Cu") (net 4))
 (segment (start 95.5 81.05) (end 130.9 81.05) (width 0.5) (layer "F.Cu") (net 4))
 (segment (start 74.5 81.05) (end 74.5 79.05) (width 0.5) (layer "F.Cu") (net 4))
 (segment (start 95.5 79.05) (end 95.5 81.05) (width 0.5) (layer "F.Cu") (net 4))
 (segment (start 74.5 79.05) (end 95.5 79.05) (width 0.5) (layer "F.Cu") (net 4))
 (segment (start 130.9 60.47) (end 144.64 60.47) (width 0.5) (layer "F.Cu") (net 4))
 (segment (start 68 77.9) (end 68 80.05) (width 0.5) (layer "F.Cu") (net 17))
 (segment (start 96.5 80.05) (end 129.4 80.05) (width 0.5) (layer "F.Cu") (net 17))
 (segment (start 68 80.05) (end 73.5 80.05) (width 0.5) (layer "F.Cu") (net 17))
 (segment (start 129.4 80.05) (end 129.4 78.25) (width 0.5) (layer "F.Cu") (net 17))
 (segment (start 96.5 78.05) (end 96.5 80.05) (width 0.5) (layer "F.Cu") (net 17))
 (segment (start 73.5 80.05) (end 73.5 78.05) (width 0.5) (layer "F.Cu") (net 17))
 (segment (start 73.5 78.05) (end 96.5 78.05) (width 0.5) (layer "F.Cu") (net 17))
 (segment (start 119 77.9) (end 119 79.05) (width 0.5) (layer "F.Cu") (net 16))
 (segment (start 127.9 75.71) (end 129.4 75.71) (width 0.5) (layer "F.Cu") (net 16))
 (segment (start 119 79.05) (end 127.9 79.05) (width 0.5) (layer "F.Cu") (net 16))
 (segment (start 127.9 79.05) (end 127.9 75.71) (width 0.5) (layer "F.Cu") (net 16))
 (segment (start 53.75 95.05) (end 59.5 95.05) (width 0.5) (layer "F.Cu") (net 21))
 (segment (start 131.9 63.01) (end 144.64 63.01) (width 0.5) (layer "F.Cu") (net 21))
 (segment (start 59.5 95.05) (end 59.5 82.05) (width 0.5) (layer "F.Cu") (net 21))
 (segment (start 53.75 107.9) (end 53.75 95.05) (width 0.5) (layer "F.Cu") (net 21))
 (segment (start 75.5 82.05) (end 75.5 80.05) (width 0.5) (layer "F.Cu") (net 21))
 (segment (start 131.9 82.05) (end 131.9 63.01) (width 0.5) (layer "F.Cu") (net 21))
 (segment (start 94.5 82.05) (end 131.9 82.05) (width 0.5) (layer "F.Cu") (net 21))
 (segment (start 94.5 80.05) (end 94.5 82.05) (width 0.5) (layer "F.Cu") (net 21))
 (segment (start 75.5 80.05) (end 94.5 80.05) (width 0.5) (layer "F.Cu") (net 21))
 (segment (start 51 107.9) (end 53.75 107.9) (width 0.5) (layer "F.Cu") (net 21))
 (segment (start 59.5 82.05) (end 75.5 82.05) (width 0.5) (layer "F.Cu") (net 21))
 (segment (start 93.5 81.05) (end 93.5 83.05) (width 0.5) (layer "F.Cu") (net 20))
 (segment (start 68 94.9) (end 70.75 94.9) (width 0.5) (layer "F.Cu") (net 20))
 (segment (start 70.75 83.05) (end 76.5 83.05) (width 0.5) (layer "F.Cu") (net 20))
 (segment (start 76.5 83.05) (end 76.5 81.05) (width 0.5) (layer "F.Cu") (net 20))
 (segment (start 93.5 83.05) (end 132.9 83.05) (width 0.5) (layer "F.Cu") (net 20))
 (segment (start 132.9 83.05) (end 132.9 65.55) (width 0.5) (layer "F.Cu") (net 20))
 (segment (start 70.75 94.9) (end 70.75 83.05) (width 0.5) (layer "F.Cu") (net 20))
 (segment (start 132.9 65.55) (end 144.64 65.55) (width 0.5) (layer "F.Cu") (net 20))
 (segment (start 76.5 81.05) (end 93.5 81.05) (width 0.5) (layer "F.Cu") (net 20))
 (segment (start 85 89.9) (end 93.5 89.9) (width 0.5) (layer "F.Cu") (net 6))
 (segment (start 133.9 68.09) (end 144.64 68.09) (width 0.5) (layer "F.Cu") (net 6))
 (segment (start 93.5 84.05) (end 133.9 84.05) (width 0.5) (layer "F.Cu") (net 6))
 (segment (start 133.9 84.05) (end 133.9 68.09) (width 0.5) (layer "F.Cu") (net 6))
 (segment (start 93.5 89.9) (end 93.5 84.05) (width 0.5) (layer "F.Cu") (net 6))
 (segment (start 134.9 85.05) (end 134.9 70.63) (width 0.5) (layer "F.Cu") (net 5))
 (segment (start 104.75 85.05) (end 134.9 85.05) (width 0.5) (layer "F.Cu") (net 5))
 (segment (start 102 94.9) (end 104.75 94.9) (width 0.5) (layer "F.Cu") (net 5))
 (segment (start 134.9 70.63) (end 144.64 70.63) (width 0.5) (layer "F.Cu") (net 5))
 (segment (start 104.75 94.9) (end 104.75 85.05) (width 0.5) (layer "F.Cu") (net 5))
 (segment (start 135.9 86.05) (end 135.9 73.17) (width 0.5) (layer "F.Cu") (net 3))
 (segment (start 129 94.9) (end 129 86.05) (width 0.5) (layer "F.Cu") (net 3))
 (segment (start 119 94.9) (end 129 94.9) (width 0.5) (layer "F.Cu") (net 3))
 (segment (start 135.9 73.17) (end 144.64 73.17) (width 0.5) (layer "F.Cu") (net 3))
 (segment (start 129 86.05) (end 135.9 86.05) (width 0.5) (layer "F.Cu") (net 3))
 (segment (start 130 87.05) (end 130 111.9) (width 0.5) (layer "F.Cu") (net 19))
 (segment (start 136.9 87.05) (end 130 87.05) (width 0.5) (layer "F.Cu") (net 19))
 (segment (start 144.64 75.71) (end 136.9 75.71) (width 0.5) (layer "F.Cu") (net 19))
 (segment (start 136.9 75.71) (end 136.9 87.05) (width 0.5) (layer "F.Cu") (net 19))
 (segment (start 122 111.9) (end 130 111.9) (width 0.5) (layer "F.Cu") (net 19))
 (segment (start 131 111.9) (end 139 111.9) (width 0.5) (layer "F.Cu") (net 18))
 (segment (start 131 88.05) (end 137.9 88.05) (width 0.5) (layer "F.Cu") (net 18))
 (segment (start 144.64 78.25) (end 137.9 78.25) (width 0.5) (layer "F.Cu") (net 18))
 (segment (start 137.9 78.25) (end 137.9 88.05) (width 0.5) (layer "F.Cu") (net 18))
 (segment (start 131 88.05) (end 131 111.9) (width 0.5) (layer "F.Cu") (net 18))
 (segment (start 139.65 55.39) (end 144.64 55.39) (width 0.5) (layer "B.Cu") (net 7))
 (segment (start 139.65 80.5) (end 139.65 87) (width 0.5) (layer "B.Cu") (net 7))
 (segment (start 139.65 80.5) (end 139.65 55.39) (width 0.5) (layer "B.Cu") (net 7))
 (segment (start 137.4 52.85) (end 137.4 89.5) (width 0.5) (layer "B.Cu") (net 9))
 (segment (start 137.4 89.5) (end 137.4 96) (width 0.5) (layer "B.Cu") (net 9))
 (segment (start 137.4 89.5) (end 138.6 89.5) (width 0.5) (layer "B.Cu") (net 9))
 (segment (start 129.4 52.85) (end 137.4 52.85) (width 0.5) (layer "B.Cu") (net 9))
 (segment (start 137.4 96) (end 138.6 96) (width 0.5) (layer "B.Cu") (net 9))
 (segment (start 141.7 92.75) (end 141.7 96) (width 0.5) (layer "F.Cu") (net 10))
 (segment (start 133.4 92.75) (end 141.7 92.75) (width 0.5) (layer "F.Cu") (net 10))
 (segment (start 133.4 91.5) (end 133.4 92.75) (width 0.5) (layer "F.Cu") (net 10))
 (segment (start 141.7 92.75) (end 141.7 89.5) (width 0.5) (layer "F.Cu") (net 10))
 (segment (start 133.4 92.75) (end 133.4 94) (width 0.5) (layer "F.Cu") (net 10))
 (segment (start 141.9 57.93) (end 141.9 89.5) (width 0.5) (layer "B.Cu") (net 10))
 (segment (start 144.64 57.93) (end 141.9 57.93) (width 0.5) (layer "B.Cu") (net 10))
 (segment (start 140.83 47.77) (end 140.83 50.31) (width 0.5) (layer "F.Cu") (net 22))
 (segment (start 140.83 50.31) (end 144.64 50.31) (width 0.5) (layer "F.Cu") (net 22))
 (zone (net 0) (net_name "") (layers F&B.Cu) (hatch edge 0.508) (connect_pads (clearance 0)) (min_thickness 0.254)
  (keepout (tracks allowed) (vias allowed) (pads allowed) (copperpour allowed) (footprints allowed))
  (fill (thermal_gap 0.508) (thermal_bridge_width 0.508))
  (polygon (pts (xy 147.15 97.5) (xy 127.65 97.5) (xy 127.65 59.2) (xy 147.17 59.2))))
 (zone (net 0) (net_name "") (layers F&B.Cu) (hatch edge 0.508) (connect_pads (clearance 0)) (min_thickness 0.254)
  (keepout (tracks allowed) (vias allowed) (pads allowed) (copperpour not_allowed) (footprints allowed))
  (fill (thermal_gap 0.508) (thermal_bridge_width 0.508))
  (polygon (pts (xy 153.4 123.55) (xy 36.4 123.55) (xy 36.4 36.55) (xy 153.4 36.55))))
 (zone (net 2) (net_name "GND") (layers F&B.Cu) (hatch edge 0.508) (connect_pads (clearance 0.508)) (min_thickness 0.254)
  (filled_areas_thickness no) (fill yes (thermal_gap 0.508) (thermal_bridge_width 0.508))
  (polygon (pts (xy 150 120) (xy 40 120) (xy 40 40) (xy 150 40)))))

